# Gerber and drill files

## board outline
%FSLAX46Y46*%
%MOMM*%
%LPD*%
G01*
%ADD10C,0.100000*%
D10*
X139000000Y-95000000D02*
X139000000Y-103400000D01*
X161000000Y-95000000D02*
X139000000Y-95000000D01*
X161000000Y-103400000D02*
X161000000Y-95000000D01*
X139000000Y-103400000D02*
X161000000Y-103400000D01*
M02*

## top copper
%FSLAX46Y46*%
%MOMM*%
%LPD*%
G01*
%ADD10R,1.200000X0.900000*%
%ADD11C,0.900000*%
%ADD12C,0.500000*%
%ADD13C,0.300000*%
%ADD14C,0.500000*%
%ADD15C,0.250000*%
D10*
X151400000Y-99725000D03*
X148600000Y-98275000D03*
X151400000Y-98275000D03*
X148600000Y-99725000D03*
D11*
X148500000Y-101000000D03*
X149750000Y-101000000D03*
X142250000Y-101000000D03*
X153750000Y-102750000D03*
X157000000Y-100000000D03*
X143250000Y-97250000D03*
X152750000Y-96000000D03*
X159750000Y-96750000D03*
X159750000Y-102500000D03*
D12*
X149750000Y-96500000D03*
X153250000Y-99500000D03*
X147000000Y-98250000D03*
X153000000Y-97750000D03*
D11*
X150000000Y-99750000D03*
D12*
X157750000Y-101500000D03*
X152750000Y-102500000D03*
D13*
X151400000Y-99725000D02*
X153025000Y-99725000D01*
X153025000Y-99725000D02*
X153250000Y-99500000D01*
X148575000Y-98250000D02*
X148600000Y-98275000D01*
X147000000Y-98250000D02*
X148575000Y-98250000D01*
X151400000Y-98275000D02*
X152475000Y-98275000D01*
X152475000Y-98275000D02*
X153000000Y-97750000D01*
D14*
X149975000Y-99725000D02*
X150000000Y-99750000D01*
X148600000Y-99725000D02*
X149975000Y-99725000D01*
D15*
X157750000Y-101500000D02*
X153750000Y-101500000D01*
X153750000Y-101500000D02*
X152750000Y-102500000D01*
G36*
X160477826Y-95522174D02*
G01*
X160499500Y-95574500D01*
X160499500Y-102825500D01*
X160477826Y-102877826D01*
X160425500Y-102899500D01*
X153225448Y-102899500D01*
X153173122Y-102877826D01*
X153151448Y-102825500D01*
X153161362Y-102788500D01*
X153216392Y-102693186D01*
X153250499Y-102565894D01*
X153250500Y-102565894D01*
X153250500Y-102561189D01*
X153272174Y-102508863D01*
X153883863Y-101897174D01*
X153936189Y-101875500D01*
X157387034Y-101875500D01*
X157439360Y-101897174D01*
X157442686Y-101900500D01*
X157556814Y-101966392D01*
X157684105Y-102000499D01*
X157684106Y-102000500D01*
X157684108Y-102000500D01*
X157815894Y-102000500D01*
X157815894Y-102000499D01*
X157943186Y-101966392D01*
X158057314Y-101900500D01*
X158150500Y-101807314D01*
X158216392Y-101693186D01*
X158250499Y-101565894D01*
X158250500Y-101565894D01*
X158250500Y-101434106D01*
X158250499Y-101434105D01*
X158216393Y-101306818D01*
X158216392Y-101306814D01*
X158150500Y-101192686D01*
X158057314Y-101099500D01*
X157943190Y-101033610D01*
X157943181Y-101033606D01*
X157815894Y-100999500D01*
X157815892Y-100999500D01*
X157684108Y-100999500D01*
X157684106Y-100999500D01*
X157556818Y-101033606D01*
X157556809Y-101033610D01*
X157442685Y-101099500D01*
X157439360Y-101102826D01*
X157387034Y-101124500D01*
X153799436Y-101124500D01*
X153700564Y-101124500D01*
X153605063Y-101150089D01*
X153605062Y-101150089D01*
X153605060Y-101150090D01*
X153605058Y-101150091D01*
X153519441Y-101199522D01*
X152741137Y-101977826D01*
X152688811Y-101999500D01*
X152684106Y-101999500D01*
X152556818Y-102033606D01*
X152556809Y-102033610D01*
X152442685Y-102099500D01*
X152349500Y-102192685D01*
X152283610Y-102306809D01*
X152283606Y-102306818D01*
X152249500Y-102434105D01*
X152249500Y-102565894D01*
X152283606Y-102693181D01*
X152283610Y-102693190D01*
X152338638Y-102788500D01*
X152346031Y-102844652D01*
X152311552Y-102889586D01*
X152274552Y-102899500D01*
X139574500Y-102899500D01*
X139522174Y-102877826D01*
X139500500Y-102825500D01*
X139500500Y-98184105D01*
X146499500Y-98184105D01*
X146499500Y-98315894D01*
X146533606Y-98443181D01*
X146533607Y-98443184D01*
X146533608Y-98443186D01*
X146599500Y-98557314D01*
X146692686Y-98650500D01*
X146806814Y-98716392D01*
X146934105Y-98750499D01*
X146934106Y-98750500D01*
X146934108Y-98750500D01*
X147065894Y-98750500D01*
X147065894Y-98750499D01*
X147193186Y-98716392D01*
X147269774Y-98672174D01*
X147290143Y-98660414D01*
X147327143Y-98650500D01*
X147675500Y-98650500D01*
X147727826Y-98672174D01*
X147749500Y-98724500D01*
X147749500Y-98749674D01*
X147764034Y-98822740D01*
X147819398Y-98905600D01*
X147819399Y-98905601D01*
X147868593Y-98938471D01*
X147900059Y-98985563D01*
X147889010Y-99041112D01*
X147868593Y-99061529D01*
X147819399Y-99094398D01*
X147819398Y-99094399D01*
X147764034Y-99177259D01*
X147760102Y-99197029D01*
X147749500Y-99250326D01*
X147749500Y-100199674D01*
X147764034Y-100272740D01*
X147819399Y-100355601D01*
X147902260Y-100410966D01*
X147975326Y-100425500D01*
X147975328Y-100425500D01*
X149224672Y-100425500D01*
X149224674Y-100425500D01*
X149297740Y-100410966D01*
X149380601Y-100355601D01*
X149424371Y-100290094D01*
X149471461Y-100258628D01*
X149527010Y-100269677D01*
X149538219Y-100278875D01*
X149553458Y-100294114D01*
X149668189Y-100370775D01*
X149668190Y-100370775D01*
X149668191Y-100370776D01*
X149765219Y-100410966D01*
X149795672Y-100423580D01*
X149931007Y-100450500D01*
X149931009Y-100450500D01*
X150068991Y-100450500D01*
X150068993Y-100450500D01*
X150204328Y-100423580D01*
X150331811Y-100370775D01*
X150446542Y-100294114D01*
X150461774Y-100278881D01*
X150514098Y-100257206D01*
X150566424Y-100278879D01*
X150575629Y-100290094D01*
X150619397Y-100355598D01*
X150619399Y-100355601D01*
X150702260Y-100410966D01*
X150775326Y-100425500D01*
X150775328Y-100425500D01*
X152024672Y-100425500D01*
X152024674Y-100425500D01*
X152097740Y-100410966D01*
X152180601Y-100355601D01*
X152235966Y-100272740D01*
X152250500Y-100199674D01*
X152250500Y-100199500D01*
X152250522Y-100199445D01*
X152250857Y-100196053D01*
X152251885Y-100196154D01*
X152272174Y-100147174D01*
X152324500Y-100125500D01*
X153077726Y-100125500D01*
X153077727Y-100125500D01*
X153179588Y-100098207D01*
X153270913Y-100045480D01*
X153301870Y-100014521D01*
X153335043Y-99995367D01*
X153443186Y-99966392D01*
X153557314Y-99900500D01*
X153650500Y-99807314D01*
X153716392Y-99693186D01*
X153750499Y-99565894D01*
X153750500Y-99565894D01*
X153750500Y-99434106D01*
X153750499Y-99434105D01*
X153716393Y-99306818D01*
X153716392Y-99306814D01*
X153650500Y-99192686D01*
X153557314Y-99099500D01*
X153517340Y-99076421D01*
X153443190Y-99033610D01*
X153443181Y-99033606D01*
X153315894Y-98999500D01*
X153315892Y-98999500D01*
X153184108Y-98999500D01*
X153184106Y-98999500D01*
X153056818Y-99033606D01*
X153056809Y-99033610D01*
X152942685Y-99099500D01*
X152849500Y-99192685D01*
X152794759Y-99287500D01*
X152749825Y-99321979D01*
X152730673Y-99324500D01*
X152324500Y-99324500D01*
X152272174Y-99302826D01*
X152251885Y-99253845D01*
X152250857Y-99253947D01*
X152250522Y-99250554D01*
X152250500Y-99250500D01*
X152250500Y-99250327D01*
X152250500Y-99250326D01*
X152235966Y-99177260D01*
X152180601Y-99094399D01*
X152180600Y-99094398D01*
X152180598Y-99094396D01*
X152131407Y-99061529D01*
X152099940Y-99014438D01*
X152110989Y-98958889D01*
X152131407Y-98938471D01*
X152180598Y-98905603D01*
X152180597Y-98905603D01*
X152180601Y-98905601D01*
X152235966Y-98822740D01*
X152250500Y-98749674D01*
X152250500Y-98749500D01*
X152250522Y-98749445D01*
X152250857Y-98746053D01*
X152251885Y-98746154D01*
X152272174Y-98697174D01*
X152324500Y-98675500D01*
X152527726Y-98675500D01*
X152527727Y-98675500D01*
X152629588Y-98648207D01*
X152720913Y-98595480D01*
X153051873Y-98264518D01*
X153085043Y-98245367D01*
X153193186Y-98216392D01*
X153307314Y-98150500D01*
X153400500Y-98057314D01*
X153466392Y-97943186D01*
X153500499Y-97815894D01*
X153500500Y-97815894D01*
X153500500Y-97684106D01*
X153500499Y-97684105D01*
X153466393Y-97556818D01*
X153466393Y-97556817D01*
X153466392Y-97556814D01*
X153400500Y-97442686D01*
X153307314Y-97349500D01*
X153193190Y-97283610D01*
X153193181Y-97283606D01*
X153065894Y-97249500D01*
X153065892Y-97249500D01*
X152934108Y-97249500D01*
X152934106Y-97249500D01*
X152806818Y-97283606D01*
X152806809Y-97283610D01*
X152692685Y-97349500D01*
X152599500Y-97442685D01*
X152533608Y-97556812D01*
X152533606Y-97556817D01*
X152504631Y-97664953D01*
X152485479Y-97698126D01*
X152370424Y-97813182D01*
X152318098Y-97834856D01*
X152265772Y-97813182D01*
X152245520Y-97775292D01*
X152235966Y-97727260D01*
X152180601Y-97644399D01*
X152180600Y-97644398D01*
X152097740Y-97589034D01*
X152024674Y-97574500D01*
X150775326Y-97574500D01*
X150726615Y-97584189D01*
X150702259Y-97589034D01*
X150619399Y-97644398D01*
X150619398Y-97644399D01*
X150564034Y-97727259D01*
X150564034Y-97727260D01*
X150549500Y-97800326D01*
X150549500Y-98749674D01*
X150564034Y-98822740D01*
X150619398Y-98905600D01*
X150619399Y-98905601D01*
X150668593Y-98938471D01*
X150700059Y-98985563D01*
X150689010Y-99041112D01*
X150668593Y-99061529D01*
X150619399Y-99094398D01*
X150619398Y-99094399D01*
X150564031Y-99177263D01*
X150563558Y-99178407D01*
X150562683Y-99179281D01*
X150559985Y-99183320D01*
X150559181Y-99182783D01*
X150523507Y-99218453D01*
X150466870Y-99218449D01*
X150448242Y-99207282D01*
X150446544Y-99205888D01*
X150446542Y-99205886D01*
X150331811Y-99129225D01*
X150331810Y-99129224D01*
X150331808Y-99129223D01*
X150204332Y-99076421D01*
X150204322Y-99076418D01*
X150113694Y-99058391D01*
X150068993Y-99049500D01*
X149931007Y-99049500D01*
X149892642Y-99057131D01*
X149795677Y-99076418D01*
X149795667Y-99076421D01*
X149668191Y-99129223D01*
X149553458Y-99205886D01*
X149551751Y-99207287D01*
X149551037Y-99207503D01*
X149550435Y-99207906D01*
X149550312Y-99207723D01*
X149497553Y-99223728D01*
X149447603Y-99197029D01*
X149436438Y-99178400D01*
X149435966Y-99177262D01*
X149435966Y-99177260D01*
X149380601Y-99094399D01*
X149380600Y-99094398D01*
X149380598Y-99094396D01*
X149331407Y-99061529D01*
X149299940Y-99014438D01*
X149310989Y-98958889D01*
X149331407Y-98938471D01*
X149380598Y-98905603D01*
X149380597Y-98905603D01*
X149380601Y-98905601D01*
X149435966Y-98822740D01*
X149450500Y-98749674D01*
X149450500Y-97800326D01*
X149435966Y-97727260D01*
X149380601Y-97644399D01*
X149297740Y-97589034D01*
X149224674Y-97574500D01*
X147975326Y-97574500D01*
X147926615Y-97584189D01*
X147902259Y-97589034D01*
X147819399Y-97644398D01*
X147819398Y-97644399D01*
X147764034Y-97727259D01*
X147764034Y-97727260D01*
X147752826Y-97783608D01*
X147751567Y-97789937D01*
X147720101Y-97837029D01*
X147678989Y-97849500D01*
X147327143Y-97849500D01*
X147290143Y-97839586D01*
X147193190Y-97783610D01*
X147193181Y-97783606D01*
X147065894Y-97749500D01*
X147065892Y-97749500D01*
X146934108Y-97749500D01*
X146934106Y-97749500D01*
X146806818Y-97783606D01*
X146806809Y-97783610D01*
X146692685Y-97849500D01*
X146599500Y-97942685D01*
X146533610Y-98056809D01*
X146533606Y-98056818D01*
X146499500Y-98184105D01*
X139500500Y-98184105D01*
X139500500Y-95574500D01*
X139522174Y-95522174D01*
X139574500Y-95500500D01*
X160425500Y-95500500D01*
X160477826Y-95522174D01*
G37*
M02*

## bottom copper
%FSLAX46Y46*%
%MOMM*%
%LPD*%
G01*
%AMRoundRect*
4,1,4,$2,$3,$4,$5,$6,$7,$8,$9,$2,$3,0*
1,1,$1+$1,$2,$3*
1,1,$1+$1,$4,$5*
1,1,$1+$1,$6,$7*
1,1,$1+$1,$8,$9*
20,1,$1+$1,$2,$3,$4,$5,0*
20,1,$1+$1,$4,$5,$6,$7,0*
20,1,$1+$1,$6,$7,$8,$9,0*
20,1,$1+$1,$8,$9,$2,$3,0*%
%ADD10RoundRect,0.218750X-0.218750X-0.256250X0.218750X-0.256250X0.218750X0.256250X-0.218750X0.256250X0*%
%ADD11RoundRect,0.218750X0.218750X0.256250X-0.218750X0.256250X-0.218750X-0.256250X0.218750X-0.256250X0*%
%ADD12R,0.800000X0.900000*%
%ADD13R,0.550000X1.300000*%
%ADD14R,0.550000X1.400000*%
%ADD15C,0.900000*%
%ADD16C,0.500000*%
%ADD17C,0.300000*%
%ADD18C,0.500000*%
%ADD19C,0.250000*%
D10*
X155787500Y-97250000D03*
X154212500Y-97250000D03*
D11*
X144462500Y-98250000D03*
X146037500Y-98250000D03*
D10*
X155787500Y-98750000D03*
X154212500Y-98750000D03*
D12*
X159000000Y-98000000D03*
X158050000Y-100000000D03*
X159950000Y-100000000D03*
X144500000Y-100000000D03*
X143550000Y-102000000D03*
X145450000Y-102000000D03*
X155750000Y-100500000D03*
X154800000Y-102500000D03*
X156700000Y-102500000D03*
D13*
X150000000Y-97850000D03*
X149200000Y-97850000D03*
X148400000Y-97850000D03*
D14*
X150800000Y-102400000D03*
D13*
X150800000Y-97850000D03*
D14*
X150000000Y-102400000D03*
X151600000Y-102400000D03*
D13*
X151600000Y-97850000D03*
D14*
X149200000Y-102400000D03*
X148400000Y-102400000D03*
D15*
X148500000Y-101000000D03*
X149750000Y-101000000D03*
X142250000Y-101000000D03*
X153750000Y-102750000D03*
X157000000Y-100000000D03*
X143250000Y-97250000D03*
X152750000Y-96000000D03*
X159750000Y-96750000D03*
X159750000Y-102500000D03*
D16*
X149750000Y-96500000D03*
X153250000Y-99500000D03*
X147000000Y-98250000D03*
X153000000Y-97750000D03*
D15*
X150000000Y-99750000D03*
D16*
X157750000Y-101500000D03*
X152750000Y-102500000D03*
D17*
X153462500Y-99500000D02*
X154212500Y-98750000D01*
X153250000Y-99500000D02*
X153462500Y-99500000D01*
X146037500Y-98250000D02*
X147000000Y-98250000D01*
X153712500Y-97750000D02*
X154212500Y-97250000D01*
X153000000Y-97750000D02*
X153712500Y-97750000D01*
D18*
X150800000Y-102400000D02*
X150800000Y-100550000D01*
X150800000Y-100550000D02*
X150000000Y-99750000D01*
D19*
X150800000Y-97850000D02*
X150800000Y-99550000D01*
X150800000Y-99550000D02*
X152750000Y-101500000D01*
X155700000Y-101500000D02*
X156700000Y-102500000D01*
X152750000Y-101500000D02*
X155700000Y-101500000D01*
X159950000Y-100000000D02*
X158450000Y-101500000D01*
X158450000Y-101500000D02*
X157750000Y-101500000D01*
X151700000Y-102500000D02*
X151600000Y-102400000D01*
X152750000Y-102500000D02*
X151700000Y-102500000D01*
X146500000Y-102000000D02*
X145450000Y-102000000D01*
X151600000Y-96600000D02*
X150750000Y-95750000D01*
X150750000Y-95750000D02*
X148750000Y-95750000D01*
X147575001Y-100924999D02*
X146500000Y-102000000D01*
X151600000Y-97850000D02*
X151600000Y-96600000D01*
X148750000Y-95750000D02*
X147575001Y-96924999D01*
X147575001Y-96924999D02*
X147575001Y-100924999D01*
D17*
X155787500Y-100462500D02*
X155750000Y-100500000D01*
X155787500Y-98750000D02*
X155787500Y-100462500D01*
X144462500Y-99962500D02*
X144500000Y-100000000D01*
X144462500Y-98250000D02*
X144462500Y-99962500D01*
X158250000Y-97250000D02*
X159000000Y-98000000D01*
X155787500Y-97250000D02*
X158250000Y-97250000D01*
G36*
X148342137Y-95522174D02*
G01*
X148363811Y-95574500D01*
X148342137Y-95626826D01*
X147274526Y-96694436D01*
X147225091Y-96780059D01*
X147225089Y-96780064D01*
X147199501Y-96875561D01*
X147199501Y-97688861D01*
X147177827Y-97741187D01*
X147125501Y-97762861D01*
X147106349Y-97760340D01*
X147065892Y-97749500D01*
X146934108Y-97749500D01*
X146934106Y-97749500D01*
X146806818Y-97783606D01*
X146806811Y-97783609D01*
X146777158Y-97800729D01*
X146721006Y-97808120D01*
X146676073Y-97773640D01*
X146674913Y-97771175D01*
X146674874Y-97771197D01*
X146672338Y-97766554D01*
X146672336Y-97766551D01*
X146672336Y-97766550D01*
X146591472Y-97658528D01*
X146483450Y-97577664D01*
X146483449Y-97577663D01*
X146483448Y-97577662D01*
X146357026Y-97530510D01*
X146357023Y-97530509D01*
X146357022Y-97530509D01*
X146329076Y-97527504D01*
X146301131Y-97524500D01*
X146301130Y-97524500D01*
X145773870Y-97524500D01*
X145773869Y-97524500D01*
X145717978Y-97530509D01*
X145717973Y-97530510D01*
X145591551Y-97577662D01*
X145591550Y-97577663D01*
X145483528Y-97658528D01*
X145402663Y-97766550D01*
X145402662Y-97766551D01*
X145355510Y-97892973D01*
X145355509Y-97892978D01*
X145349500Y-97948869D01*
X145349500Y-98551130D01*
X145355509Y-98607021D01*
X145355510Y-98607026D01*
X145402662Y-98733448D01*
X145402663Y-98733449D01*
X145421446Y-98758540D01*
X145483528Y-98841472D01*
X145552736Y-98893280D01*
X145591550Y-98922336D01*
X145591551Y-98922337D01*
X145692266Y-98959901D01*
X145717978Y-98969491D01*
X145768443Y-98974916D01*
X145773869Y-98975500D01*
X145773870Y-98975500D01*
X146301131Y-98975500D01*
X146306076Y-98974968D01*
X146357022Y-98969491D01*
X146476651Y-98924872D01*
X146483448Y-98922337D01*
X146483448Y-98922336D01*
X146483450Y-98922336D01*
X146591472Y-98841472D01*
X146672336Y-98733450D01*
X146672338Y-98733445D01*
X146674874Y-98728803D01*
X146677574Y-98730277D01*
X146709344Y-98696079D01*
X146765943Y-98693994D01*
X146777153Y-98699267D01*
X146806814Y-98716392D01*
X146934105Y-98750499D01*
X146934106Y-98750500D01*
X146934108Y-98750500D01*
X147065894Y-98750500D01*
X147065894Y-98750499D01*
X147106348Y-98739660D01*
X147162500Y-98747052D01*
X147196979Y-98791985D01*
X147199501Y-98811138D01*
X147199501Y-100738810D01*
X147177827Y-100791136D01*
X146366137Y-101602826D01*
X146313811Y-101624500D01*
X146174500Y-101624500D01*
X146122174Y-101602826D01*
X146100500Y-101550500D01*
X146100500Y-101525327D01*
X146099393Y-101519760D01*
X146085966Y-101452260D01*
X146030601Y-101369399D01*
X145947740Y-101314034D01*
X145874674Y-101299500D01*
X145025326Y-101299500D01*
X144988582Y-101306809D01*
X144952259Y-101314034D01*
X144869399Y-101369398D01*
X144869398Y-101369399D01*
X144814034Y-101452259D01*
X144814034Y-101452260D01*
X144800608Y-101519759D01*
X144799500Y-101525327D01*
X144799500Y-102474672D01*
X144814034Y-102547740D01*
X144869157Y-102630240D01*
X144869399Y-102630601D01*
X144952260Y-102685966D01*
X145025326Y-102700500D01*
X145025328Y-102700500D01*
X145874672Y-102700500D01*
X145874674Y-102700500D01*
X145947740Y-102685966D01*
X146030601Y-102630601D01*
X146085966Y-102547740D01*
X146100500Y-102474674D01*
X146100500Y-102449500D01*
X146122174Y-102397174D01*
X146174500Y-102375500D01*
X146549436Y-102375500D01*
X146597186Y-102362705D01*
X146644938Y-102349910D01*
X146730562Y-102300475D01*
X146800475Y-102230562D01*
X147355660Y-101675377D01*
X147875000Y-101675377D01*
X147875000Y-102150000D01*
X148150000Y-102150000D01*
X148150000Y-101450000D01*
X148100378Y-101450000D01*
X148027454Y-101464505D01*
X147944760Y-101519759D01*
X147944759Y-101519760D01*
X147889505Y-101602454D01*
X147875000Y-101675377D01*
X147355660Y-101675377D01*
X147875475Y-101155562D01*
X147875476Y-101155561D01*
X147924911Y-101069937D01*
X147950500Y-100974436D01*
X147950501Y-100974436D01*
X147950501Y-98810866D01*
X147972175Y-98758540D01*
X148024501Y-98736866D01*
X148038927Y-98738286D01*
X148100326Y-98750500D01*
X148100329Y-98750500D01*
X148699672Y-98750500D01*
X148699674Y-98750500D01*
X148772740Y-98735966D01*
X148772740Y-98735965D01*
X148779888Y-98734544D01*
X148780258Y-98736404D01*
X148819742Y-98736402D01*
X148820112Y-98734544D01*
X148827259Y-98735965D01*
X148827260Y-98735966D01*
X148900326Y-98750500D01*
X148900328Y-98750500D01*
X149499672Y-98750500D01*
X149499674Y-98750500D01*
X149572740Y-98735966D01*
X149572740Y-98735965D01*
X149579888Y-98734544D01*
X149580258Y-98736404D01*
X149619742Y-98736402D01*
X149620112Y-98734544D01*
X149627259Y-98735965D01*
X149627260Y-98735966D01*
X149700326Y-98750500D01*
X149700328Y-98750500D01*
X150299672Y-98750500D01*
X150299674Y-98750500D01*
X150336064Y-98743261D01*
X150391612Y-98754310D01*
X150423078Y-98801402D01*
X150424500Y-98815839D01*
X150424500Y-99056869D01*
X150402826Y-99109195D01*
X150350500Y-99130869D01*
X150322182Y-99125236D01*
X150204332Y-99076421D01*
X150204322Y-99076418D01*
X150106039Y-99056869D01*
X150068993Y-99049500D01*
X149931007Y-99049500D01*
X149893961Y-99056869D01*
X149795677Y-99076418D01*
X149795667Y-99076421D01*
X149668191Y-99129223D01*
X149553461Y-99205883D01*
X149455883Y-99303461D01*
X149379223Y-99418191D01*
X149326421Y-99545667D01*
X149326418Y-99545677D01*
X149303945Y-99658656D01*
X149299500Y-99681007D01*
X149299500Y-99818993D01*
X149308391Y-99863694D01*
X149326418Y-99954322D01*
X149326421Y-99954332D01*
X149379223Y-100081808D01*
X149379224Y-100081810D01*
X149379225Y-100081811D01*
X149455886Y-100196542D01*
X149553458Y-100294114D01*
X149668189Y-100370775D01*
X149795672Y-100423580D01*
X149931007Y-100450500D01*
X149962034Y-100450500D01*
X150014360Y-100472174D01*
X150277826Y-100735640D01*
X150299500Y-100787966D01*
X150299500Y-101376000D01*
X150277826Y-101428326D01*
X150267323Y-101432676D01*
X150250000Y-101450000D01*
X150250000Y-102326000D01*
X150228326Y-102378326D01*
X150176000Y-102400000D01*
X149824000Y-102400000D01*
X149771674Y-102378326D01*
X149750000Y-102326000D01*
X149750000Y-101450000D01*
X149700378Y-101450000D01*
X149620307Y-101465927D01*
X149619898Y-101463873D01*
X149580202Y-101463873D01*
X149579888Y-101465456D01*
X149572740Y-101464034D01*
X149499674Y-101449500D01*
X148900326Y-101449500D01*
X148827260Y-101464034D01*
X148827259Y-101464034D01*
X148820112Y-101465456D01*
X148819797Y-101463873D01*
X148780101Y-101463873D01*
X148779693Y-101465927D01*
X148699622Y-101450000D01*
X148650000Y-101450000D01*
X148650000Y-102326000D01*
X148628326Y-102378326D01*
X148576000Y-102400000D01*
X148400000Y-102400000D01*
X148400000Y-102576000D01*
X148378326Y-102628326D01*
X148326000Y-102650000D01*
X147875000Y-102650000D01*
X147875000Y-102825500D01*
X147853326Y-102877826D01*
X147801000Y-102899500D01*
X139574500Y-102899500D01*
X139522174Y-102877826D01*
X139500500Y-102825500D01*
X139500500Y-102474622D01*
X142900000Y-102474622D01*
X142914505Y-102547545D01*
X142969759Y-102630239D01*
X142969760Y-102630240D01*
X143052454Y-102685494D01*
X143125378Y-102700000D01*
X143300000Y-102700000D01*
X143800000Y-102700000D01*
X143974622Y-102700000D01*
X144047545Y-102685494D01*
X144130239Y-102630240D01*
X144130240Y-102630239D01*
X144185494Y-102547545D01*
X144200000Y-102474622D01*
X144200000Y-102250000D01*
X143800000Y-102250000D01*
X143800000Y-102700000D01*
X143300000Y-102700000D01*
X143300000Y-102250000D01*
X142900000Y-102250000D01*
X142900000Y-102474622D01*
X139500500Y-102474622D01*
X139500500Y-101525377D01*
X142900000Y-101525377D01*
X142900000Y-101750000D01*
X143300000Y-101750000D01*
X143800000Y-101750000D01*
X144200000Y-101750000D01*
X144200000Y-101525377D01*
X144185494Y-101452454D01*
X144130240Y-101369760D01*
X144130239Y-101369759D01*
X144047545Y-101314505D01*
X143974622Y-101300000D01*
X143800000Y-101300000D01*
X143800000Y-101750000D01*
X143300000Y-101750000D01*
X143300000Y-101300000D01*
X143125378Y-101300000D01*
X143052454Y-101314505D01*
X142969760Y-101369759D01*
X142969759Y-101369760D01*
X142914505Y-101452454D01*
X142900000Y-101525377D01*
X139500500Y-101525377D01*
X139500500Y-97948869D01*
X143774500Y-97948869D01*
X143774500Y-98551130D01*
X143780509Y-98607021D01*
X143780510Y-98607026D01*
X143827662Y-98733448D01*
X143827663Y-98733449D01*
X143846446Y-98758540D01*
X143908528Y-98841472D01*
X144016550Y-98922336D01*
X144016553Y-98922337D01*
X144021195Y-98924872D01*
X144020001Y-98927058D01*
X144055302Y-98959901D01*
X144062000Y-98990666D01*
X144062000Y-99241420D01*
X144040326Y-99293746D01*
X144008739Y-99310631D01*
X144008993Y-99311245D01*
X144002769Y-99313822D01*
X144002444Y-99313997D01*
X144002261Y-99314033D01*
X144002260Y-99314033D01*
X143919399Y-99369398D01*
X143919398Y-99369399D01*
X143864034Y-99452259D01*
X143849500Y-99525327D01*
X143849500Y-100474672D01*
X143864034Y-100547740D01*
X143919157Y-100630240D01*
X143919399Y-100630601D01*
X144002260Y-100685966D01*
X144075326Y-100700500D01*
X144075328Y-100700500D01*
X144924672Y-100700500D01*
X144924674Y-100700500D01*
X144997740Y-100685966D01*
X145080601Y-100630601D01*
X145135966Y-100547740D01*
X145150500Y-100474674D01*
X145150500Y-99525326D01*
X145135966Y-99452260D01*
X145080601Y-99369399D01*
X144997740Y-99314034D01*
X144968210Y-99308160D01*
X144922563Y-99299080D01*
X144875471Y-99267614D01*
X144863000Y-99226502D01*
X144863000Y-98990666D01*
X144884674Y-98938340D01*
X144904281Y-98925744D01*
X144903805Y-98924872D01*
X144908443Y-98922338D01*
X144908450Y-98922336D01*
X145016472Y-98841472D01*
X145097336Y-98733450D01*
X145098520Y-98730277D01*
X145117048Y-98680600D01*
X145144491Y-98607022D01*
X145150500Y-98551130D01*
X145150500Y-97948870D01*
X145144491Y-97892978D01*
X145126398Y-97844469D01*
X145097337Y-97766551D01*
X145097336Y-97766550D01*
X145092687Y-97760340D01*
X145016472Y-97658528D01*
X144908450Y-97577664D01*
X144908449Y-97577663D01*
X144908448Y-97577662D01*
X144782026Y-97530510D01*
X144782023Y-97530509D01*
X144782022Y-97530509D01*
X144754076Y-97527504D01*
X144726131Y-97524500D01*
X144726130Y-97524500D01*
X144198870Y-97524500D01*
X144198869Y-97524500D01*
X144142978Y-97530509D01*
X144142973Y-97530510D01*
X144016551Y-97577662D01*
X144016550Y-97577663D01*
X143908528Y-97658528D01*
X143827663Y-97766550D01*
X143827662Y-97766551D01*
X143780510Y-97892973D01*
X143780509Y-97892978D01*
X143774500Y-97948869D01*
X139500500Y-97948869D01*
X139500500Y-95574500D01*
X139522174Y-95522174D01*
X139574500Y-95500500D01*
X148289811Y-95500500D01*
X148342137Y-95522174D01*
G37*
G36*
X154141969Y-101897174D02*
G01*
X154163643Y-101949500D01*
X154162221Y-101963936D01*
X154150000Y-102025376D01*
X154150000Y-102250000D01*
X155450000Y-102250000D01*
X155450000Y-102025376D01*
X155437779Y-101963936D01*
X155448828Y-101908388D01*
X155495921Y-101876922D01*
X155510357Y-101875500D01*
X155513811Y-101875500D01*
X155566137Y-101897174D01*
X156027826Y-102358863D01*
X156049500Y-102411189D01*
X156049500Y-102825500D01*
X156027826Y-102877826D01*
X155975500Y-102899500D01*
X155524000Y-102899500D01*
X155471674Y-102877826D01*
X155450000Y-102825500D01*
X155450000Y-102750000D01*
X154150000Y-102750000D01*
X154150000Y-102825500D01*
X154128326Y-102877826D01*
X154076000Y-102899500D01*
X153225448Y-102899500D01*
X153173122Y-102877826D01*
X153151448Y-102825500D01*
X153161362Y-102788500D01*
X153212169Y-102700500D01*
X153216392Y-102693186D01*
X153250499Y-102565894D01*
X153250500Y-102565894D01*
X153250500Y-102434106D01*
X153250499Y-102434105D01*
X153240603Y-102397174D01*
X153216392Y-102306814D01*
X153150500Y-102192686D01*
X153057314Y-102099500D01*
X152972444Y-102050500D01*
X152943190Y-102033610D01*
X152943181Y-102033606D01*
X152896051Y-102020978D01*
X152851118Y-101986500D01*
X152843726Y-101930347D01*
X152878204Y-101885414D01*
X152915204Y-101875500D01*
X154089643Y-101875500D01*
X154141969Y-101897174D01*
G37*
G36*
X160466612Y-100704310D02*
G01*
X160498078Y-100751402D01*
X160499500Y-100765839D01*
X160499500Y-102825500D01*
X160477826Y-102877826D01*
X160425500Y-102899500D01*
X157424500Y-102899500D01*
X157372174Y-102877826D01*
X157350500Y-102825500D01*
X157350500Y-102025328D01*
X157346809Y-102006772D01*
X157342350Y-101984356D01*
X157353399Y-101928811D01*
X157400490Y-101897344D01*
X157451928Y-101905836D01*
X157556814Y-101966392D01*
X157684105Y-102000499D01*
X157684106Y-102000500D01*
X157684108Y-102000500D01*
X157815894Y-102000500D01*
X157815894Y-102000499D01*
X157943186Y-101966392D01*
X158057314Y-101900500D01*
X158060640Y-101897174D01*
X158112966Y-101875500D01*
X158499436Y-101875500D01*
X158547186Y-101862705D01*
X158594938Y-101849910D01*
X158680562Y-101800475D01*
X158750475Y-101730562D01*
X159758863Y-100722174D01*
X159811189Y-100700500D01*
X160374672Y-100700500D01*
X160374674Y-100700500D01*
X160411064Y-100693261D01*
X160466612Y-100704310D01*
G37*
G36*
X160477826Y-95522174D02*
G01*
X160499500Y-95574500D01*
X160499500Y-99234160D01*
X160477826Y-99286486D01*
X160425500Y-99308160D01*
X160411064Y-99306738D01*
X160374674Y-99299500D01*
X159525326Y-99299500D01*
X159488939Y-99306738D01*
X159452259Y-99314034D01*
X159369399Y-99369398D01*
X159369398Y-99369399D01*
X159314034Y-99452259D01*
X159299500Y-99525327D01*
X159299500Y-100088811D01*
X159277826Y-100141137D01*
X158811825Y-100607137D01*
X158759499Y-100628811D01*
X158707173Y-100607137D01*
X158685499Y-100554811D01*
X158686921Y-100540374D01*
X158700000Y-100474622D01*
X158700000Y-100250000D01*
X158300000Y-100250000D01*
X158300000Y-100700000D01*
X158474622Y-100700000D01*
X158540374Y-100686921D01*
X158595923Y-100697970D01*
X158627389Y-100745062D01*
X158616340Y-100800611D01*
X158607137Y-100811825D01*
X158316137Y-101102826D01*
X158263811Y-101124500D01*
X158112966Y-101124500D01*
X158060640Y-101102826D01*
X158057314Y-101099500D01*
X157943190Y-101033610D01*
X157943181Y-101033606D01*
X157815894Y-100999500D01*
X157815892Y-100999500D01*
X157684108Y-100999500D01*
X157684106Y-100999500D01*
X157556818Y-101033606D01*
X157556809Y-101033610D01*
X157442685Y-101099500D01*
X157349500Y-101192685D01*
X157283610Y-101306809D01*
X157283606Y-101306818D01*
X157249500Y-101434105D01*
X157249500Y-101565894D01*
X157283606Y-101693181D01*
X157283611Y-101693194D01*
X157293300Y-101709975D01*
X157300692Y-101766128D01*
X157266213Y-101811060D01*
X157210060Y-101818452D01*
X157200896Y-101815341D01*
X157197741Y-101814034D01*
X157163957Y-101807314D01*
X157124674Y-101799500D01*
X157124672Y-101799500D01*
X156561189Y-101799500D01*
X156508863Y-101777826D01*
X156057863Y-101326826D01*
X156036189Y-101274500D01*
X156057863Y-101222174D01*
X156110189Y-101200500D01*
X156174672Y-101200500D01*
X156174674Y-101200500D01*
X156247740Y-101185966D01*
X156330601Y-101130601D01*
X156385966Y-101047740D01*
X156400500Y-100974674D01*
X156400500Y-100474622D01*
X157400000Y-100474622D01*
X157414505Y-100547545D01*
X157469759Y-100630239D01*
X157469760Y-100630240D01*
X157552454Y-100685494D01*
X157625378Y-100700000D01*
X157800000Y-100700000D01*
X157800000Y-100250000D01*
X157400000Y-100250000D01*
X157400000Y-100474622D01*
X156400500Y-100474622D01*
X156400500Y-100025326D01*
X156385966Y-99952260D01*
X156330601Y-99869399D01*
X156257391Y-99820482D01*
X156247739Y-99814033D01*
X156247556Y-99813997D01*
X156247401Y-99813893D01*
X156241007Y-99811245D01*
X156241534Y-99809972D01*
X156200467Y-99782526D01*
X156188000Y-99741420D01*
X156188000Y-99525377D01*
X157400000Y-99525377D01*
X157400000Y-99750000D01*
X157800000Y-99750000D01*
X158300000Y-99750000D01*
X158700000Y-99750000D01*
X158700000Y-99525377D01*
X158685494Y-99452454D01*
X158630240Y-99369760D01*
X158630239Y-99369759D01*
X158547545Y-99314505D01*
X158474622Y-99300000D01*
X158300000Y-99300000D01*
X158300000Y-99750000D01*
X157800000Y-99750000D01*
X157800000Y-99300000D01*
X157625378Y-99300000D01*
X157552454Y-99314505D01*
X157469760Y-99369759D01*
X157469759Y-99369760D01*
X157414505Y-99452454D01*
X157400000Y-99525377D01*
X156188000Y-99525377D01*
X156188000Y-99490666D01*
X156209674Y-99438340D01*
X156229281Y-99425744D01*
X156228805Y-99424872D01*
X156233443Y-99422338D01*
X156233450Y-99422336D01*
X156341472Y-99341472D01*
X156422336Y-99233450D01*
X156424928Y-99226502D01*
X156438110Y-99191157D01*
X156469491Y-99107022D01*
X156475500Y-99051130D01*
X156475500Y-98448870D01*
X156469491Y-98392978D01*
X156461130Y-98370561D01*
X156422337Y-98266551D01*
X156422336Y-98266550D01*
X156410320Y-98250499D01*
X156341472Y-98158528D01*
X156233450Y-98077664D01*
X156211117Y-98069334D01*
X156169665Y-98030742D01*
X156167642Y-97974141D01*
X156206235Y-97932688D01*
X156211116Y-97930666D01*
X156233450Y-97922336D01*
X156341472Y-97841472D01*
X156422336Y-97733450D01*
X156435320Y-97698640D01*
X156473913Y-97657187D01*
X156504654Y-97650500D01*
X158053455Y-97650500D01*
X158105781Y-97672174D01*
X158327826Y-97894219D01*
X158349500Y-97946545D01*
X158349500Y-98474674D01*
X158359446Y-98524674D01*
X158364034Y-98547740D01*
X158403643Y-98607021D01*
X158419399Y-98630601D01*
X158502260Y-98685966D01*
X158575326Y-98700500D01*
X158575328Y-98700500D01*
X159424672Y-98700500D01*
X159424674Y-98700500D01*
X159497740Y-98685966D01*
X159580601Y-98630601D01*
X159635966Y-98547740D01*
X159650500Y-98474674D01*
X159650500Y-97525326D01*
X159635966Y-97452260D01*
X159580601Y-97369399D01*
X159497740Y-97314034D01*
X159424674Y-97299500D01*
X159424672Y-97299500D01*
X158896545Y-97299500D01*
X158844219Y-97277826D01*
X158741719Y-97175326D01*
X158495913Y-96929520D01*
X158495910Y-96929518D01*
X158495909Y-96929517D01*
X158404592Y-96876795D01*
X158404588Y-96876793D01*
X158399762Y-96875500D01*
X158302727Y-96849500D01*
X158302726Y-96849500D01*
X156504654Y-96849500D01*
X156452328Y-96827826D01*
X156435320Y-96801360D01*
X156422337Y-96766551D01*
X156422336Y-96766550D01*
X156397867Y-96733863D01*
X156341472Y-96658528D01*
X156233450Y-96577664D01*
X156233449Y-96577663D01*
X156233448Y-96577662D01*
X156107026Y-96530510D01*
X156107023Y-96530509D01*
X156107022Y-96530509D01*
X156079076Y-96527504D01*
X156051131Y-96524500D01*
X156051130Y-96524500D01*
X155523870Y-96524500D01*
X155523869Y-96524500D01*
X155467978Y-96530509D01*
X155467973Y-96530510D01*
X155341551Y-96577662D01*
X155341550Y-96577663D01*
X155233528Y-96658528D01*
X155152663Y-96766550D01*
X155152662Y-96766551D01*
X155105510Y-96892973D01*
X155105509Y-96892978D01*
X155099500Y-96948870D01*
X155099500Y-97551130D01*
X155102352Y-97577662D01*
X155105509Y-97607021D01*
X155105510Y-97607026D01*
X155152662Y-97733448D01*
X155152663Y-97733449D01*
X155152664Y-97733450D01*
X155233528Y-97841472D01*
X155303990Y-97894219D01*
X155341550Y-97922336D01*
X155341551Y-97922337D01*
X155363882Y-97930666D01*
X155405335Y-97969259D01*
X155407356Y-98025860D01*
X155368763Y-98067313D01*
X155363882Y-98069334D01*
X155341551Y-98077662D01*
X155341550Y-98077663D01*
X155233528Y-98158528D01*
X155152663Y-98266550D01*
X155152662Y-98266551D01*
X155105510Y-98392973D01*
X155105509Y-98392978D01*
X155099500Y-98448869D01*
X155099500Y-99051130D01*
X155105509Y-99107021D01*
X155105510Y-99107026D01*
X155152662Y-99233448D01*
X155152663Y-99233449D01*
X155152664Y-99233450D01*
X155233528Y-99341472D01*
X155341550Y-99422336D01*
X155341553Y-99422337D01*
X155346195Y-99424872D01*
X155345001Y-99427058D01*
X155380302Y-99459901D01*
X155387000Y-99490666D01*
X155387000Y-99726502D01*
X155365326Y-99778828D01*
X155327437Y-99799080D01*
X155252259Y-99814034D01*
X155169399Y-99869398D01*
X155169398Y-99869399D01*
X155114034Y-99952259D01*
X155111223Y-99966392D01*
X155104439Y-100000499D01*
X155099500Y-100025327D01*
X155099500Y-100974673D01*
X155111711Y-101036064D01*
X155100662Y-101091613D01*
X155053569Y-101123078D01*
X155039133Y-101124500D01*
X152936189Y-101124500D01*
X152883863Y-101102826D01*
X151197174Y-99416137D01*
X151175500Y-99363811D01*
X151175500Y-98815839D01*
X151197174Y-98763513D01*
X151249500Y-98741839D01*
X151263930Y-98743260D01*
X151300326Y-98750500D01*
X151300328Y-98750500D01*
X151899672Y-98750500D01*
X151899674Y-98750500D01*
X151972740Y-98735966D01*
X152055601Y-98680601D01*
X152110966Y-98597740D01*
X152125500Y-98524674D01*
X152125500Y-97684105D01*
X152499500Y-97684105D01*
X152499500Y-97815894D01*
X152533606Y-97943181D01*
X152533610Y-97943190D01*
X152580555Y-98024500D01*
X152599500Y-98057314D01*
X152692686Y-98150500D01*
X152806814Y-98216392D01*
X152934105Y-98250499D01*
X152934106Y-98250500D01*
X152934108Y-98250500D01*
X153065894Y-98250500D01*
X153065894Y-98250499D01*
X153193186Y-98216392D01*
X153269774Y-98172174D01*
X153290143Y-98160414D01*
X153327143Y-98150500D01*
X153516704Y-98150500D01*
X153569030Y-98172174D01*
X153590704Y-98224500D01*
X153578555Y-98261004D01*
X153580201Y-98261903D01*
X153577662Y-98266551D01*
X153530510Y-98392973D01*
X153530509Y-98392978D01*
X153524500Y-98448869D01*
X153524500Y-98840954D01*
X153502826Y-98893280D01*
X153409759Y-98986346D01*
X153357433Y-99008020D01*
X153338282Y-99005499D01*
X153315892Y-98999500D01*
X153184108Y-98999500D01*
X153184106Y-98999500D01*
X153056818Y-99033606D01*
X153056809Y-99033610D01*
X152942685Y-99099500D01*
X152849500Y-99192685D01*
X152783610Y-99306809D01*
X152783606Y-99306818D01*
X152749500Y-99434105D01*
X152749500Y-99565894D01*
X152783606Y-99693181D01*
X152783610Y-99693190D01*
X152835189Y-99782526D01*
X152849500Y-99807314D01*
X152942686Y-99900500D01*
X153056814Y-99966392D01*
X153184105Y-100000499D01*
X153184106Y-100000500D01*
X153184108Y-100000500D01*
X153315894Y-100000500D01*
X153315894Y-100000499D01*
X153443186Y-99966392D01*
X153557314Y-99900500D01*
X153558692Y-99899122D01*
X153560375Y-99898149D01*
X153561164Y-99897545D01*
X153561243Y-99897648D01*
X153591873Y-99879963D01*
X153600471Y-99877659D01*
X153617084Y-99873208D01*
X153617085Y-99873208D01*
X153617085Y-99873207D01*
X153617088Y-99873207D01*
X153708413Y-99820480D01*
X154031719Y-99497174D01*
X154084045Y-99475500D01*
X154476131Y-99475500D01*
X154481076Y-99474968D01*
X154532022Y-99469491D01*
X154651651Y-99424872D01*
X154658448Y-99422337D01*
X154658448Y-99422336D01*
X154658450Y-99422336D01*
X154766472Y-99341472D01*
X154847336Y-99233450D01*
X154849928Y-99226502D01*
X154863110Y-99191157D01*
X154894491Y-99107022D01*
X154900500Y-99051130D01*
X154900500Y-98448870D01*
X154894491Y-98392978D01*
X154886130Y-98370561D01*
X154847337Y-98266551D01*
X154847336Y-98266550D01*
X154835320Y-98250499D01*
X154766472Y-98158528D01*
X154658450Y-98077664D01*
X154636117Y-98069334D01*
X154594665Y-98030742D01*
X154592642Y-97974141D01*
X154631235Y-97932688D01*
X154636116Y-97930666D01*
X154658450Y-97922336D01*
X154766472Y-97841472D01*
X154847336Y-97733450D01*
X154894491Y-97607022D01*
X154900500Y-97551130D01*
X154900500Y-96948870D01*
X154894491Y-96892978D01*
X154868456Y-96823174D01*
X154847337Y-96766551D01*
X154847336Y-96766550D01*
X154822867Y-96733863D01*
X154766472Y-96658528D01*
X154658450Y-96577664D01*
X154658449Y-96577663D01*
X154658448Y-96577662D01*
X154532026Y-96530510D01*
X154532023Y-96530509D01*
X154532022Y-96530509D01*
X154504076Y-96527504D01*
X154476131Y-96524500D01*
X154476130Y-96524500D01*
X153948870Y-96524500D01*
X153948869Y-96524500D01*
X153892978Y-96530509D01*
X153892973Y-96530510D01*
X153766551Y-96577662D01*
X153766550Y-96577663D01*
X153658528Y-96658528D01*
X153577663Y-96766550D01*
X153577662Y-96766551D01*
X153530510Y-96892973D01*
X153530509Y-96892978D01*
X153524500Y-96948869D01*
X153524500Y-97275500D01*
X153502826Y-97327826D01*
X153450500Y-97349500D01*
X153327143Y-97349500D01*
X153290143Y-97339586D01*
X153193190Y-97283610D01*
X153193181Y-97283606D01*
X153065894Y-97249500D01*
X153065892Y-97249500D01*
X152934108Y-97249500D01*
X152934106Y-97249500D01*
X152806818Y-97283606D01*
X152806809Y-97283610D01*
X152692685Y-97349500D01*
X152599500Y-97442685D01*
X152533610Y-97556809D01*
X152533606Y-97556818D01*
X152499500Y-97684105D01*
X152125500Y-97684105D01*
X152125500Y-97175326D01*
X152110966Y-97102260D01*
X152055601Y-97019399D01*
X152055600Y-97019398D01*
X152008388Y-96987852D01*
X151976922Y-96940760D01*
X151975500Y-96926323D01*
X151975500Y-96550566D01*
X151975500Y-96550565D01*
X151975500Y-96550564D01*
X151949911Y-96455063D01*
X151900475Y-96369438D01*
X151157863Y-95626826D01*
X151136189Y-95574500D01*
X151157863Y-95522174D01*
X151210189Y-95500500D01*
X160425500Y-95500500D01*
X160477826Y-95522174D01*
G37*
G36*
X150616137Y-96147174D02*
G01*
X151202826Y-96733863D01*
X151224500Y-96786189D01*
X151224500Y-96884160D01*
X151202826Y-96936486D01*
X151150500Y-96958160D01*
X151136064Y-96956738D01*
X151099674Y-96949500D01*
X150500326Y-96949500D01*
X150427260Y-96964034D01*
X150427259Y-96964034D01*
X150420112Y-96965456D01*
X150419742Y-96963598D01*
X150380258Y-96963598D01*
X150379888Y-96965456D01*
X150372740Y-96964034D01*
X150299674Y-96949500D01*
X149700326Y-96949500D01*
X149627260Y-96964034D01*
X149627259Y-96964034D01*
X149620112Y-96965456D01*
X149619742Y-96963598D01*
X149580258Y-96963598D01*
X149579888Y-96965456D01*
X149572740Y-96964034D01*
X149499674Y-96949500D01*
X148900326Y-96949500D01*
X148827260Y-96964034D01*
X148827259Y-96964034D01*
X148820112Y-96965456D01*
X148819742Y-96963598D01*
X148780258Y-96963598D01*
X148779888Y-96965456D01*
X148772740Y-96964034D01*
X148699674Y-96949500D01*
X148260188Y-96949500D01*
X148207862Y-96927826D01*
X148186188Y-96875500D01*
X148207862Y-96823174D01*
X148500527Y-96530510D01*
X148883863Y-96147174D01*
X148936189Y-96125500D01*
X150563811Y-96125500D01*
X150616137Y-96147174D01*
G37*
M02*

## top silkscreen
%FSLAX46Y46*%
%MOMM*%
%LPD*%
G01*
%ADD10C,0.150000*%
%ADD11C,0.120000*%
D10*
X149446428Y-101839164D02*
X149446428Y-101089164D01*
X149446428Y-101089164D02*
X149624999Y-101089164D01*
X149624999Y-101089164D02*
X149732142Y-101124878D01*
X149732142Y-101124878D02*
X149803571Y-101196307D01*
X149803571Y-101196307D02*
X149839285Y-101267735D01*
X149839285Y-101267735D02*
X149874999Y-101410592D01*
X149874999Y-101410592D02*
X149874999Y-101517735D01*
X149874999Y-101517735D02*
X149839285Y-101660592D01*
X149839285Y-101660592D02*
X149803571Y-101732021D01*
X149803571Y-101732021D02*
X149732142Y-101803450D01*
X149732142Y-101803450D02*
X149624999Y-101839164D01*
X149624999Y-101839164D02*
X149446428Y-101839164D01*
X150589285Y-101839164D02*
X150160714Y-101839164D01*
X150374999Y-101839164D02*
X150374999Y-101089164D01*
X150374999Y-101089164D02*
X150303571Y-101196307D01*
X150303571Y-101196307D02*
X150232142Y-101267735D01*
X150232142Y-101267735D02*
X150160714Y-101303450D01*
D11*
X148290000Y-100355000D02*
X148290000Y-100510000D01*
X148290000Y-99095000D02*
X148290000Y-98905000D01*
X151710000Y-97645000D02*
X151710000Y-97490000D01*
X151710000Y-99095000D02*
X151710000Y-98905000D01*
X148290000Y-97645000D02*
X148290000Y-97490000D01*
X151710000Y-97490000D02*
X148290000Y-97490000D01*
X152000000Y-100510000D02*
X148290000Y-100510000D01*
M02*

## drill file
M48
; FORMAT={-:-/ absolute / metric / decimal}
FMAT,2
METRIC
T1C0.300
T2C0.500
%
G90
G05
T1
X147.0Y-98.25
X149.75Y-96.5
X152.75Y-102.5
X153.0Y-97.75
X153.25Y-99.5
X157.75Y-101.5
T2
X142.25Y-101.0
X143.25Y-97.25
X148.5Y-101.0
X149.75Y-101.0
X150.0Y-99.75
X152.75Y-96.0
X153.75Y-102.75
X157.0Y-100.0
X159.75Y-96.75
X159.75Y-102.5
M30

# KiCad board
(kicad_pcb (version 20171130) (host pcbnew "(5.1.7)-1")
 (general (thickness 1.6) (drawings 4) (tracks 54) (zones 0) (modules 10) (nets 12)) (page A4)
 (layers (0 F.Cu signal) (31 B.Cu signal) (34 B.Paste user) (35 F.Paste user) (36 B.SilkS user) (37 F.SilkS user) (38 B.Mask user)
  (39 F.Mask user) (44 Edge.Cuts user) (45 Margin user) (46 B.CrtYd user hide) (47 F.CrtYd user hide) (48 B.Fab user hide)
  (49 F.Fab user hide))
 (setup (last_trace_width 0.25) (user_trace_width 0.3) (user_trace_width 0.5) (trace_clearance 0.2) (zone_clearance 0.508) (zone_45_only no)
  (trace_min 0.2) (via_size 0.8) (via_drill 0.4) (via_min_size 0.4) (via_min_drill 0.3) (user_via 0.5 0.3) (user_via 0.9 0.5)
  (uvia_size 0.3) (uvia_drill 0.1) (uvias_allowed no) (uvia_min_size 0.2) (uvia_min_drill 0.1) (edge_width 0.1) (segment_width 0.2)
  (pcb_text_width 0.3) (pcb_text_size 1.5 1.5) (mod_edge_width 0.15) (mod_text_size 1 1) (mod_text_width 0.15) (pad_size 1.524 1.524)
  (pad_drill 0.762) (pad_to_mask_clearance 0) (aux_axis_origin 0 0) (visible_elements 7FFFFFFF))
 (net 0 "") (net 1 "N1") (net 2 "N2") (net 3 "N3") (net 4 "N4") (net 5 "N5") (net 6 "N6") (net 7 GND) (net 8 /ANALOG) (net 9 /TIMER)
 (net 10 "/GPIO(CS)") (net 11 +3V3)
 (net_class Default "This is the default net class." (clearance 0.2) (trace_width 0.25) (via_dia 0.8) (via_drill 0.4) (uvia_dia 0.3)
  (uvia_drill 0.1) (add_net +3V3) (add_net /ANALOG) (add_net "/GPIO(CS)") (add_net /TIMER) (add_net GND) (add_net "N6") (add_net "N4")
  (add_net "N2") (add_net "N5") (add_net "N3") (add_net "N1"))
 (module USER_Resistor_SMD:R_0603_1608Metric (layer B.Cu) (at 155 97.25)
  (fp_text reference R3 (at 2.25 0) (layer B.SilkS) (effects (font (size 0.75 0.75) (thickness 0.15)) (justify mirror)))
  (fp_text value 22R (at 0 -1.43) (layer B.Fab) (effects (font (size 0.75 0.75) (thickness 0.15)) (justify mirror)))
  (pad 2 smd roundrect (at 0.7875 0) (size 0.875 0.95) (layers B.Cu B.Paste B.Mask) (roundrect_rratio 0.25) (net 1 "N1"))
  (pad 1 smd roundrect (at -0.7875 0) (size 0.875 0.95) (layers B.Cu B.Paste B.Mask) (roundrect_rratio 0.25) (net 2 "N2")))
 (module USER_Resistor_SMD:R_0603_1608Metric (layer B.Cu) (at 145.25 98.25 180)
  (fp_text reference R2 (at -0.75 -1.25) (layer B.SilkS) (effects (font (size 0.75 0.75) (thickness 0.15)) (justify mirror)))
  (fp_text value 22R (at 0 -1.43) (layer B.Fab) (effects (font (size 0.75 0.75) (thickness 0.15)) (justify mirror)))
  (pad 2 smd roundrect (at 0.7875 0 180) (size 0.875 0.95) (layers B.Cu B.Paste B.Mask) (roundrect_rratio 0.25) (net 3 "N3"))
  (pad 1 smd roundrect (at -0.7875 0 180) (size 0.875 0.95) (layers B.Cu B.Paste B.Mask) (roundrect_rratio 0.25) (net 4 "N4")))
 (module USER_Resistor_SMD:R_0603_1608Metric (layer B.Cu) (at 155 98.75)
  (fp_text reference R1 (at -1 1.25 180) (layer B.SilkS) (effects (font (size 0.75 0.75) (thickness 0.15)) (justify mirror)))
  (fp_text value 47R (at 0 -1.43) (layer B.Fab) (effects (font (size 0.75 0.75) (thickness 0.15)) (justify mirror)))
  (pad 2 smd roundrect (at 0.7875 0) (size 0.875 0.95) (layers B.Cu B.Paste B.Mask) (roundrect_rratio 0.25) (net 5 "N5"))
  (pad 1 smd roundrect (at -0.7875 0) (size 0.875 0.95) (layers B.Cu B.Paste B.Mask) (roundrect_rratio 0.25) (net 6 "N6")))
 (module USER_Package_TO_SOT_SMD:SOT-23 (layer B.Cu) (at 159 99 90)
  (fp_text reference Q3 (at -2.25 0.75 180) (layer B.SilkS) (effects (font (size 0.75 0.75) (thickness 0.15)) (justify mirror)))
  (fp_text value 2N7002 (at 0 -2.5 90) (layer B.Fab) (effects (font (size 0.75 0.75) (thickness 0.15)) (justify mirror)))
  (pad 3 smd rect (at 1 0 90) (size 0.9 0.8) (layers B.Cu B.Paste B.Mask) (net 1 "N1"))
  (pad 2 smd rect (at -1 -0.95 90) (size 0.9 0.8) (layers B.Cu B.Paste B.Mask) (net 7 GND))
  (pad 1 smd rect (at -1 0.95 90) (size 0.9 0.8) (layers B.Cu B.Paste B.Mask) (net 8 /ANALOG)))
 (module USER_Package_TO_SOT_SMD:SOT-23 (layer B.Cu) (at 144.5 101 90)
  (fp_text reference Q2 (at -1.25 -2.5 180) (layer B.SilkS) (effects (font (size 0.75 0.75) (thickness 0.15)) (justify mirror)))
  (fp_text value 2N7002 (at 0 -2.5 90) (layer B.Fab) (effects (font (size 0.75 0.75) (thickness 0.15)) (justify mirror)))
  (pad 3 smd rect (at 1 0 90) (size 0.9 0.8) (layers B.Cu B.Paste B.Mask) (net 3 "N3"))
  (pad 2 smd rect (at -1 -0.95 90) (size 0.9 0.8) (layers B.Cu B.Paste B.Mask) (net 7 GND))
  (pad 1 smd rect (at -1 0.95 90) (size 0.9 0.8) (layers B.Cu B.Paste B.Mask) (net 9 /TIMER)))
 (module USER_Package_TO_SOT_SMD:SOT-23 (layer B.Cu) (at 155.75 101.5 90)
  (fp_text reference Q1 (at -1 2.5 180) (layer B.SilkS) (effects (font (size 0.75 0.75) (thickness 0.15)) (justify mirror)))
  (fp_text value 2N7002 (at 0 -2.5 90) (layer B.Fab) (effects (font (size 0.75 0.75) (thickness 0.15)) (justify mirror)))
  (pad 3 smd rect (at 1 0 90) (size 0.9 0.8) (layers B.Cu B.Paste B.Mask) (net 5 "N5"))
  (pad 2 smd rect (at -1 -0.95 90) (size 0.9 0.8) (layers B.Cu B.Paste B.Mask) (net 7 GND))
  (pad 1 smd rect (at -1 0.95 90) (size 0.9 0.8) (layers B.Cu B.Paste B.Mask) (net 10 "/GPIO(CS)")))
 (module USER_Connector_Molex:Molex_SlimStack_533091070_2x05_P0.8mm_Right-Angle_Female (layer B.Cu) (at 150 100)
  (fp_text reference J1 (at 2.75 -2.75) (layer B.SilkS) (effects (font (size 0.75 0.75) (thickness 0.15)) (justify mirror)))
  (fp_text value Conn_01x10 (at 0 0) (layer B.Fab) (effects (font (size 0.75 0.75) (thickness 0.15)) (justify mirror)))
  (pad 5 smd rect (at 0 -2.15 180) (size 0.55 1.3) (layers B.Cu B.Paste B.Mask))
  (pad 3 smd rect (at -0.8 -2.15 180) (size 0.55 1.3) (layers B.Cu B.Paste B.Mask))
  (pad 1 smd rect (at -1.6 -2.15 180) (size 0.55 1.3) (layers B.Cu B.Paste B.Mask))
  (pad 8 smd rect (at 0.8 2.4 180) (size 0.55 1.4) (layers B.Cu B.Paste B.Mask) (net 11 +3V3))
  (pad 7 smd rect (at 0.8 -2.15 180) (size 0.55 1.3) (layers B.Cu B.Paste B.Mask) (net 10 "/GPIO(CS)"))
  (pad 6 smd rect (at 0 2.4 180) (size 0.55 1.4) (layers B.Cu B.Paste B.Mask) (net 7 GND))
  (pad 10 smd rect (at 1.6 2.4 180) (size 0.55 1.4) (layers B.Cu B.Paste B.Mask) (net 8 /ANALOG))
  (pad 9 smd rect (at 1.6 -2.15 180) (size 0.55 1.3) (layers B.Cu B.Paste B.Mask) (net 9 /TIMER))
  (pad 4 smd rect (at -0.8 2.4 180) (size 0.55 1.4) (layers B.Cu B.Paste B.Mask))
  (pad 2 smd rect (at -1.6 2.4 180) (size 0.55 1.4) (layers B.Cu B.Paste B.Mask) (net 7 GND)))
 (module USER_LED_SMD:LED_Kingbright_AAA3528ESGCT (layer F.Cu) (at 150 99 180)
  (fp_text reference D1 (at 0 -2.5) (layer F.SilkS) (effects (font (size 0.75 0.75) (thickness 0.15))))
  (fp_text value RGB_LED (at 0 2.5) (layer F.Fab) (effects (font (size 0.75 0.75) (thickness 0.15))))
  (fp_line (start 1.71 -1.355) (end 1.71 -1.51) (layer F.SilkS) (width 0.12))
  (fp_line (start 1.71 -0.095) (end 1.71 0.095) (layer F.SilkS) (width 0.12))
  (fp_line (start -1.71 1.355) (end -1.71 1.51) (layer F.SilkS) (width 0.12))
  (fp_line (start -1.71 -0.095) (end -1.71 0.095) (layer F.SilkS) (width 0.12))
  (fp_line (start 1.71 1.355) (end 1.71 1.51) (layer F.SilkS) (width 0.12))
  (fp_line (start -1.71 1.51) (end 1.71 1.51) (layer F.SilkS) (width 0.12))
  (fp_line (start -2 -1.51) (end 1.71 -1.51) (layer F.SilkS) (width 0.12))
  (pad 1 smd rect (at -1.4 -0.725 180) (size 1.2 0.9) (layers F.Cu F.Paste F.Mask) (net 6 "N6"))
  (pad 3 smd rect (at 1.4 0.725 180) (size 1.2 0.9) (layers F.Cu F.Paste F.Mask) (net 4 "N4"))
  (pad 4 smd rect (at -1.4 0.725 180) (size 1.2 0.9) (layers F.Cu F.Paste F.Mask) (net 2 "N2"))
  (pad 2 smd rect (at 1.4 -0.725 180) (size 1.2 0.9) (layers F.Cu F.Paste F.Mask) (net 11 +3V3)))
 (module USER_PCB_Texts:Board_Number (layer B.Cu) (at 138.9 97.4)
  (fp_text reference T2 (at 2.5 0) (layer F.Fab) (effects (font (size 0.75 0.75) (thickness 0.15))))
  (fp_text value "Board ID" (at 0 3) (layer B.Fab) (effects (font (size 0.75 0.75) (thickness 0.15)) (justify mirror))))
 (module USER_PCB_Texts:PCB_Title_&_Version (layer F.Cu) (at 147.594999 110.734999)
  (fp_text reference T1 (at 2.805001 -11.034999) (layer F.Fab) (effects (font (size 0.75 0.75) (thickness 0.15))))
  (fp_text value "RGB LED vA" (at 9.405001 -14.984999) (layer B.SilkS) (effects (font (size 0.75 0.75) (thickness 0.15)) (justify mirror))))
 (gr_line (start 139 95) (end 139 103.4) (layer Edge.Cuts) (width 0.1))
 (gr_line (start 161 95) (end 139 95) (layer Edge.Cuts) (width 0.1))
 (gr_line (start 161 103.4) (end 161 95) (layer Edge.Cuts) (width 0.1))
 (gr_line (start 139 103.4) (end 161 103.4) (layer Edge.Cuts) (width 0.1))
 (via (at 148.5 101) (size 0.9) (drill 0.5) (layers F.Cu B.Cu) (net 7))
 (via (at 149.75 101) (size 0.9) (drill 0.5) (layers F.Cu B.Cu) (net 7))
 (via (at 142.25 101) (size 0.9) (drill 0.5) (layers F.Cu B.Cu) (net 7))
 (via (at 153.75 102.75) (size 0.9) (drill 0.5) (layers F.Cu B.Cu) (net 7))
 (via (at 157 100) (size 0.9) (drill 0.5) (layers F.Cu B.Cu) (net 7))
 (via (at 143.25 97.25) (size 0.9) (drill 0.5) (layers F.Cu B.Cu) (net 7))
 (via (at 152.75 96) (size 0.9) (drill 0.5) (layers F.Cu B.Cu) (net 7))
 (via (at 159.75 96.75) (size 0.9) (drill 0.5) (layers F.Cu B.Cu) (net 7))
 (via (at 159.75 102.5) (size 0.9) (drill 0.5) (layers F.Cu B.Cu) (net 7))
 (via (at 149.75 96.5) (size 0.5) (drill 0.3) (layers F.Cu B.Cu) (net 7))
 (via (at 153.25 99.5) (size 0.5) (drill 0.3) (layers F.Cu B.Cu) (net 6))
 (segment (start 151.4 99.725) (end 153.025 99.725) (width 0.3) (layer F.Cu) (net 6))
 (segment (start 153.025 99.725) (end 153.25 99.5) (width 0.3) (layer F.Cu) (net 6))
 (segment (start 153.4625 99.5) (end 154.2125 98.75) (width 0.3) (layer B.Cu) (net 6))
 (segment (start 153.25 99.5) (end 153.4625 99.5) (width 0.3) (layer B.Cu) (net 6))
 (via (at 147 98.25) (size 0.5) (drill 0.3) (layers F.Cu B.Cu) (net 4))
 (segment (start 146.0375 98.25) (end 147 98.25) (width 0.3) (layer B.Cu) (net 4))
 (segment (start 148.575 98.25) (end 148.6 98.275) (width 0.3) (layer F.Cu) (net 4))
 (segment (start 147 98.25) (end 148.575 98.25) (width 0.3) (layer F.Cu) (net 4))
 (segment (start 151.4 98.275) (end 152.475 98.275) (width 0.3) (layer F.Cu) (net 2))
 (via (at 153 97.75) (size 0.5) (drill 0.3) (layers F.Cu B.Cu) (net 2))
 (segment (start 152.475 98.275) (end 153 97.75) (width 0.3) (layer F.Cu) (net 2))
 (segment (start 153.7125 97.75) (end 154.2125 97.25) (width 0.3) (layer B.Cu) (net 2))
 (segment (start 153 97.75) (end 153.7125 97.75) (width 0.3) (layer B.Cu) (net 2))
 (segment (start 150.8 102.4) (end 150.8 100.55) (width 0.5) (layer B.Cu) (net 11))
 (segment (start 149.975 99.725) (end 150 99.75) (width 0.5) (layer F.Cu) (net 11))
 (via (at 150 99.75) (size 0.9) (drill 0.5) (layers F.Cu B.Cu) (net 11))
 (segment (start 150.8 100.55) (end 150 99.75) (width 0.5) (layer B.Cu) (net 11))
 (segment (start 148.6 99.725) (end 149.975 99.725) (width 0.5) (layer F.Cu) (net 11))
 (segment (start 150.8 97.85) (end 150.8 99.55) (width 0.25) (layer B.Cu) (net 10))
 (segment (start 150.8 99.55) (end 152.75 101.5) (width 0.25) (layer B.Cu) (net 10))
 (segment (start 155.7 101.5) (end 156.7 102.5) (width 0.25) (layer B.Cu) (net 10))
 (segment (start 152.75 101.5) (end 155.7 101.5) (width 0.25) (layer B.Cu) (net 10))
 (via (at 157.75 101.5) (size 0.5) (drill 0.3) (layers F.Cu B.Cu) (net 8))
 (segment (start 159.95 100) (end 158.45 101.5) (width 0.25) (layer B.Cu) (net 8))
 (segment (start 158.45 101.5) (end 157.75 101.5) (width 0.25) (layer B.Cu) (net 8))
 (via (at 152.75 102.5) (size 0.5) (drill 0.3) (layers F.Cu B.Cu) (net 8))
 (segment (start 157.75 101.5) (end 153.75 101.5) (width 0.25) (layer F.Cu) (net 8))
 (segment (start 153.75 101.5) (end 152.75 102.5) (width 0.25) (layer F.Cu) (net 8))
 (segment (start 151.7 102.5) (end 151.6 102.4) (width 0.25) (layer B.Cu) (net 8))
 (segment (start 152.75 102.5) (end 151.7 102.5) (width 0.25) (layer B.Cu) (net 8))
 (segment (start 146.5 102) (end 145.45 102) (width 0.25) (layer B.Cu) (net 9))
 (segment (start 151.6 96.6) (end 150.75 95.75) (width 0.25) (layer B.Cu) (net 9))
 (segment (start 150.75 95.75) (end 148.75 95.75) (width 0.25) (layer B.Cu) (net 9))
 (segment (start 147.575001 100.924999) (end 146.5 102) (width 0.25) (layer B.Cu) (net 9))
 (segment (start 151.6 97.85) (end 151.6 96.6) (width 0.25) (layer B.Cu) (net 9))
 (segment (start 148.75 95.75) (end 147.575001 96.924999) (width 0.25) (layer B.Cu) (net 9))
 (segment (start 147.575001 96.924999) (end 147.575001 100.924999) (width 0.25) (layer B.Cu) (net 9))
 (segment (start 155.7875 100.4625) (end 155.75 100.5) (width 0.3) (layer B.Cu) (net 5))
 (segment (start 155.7875 98.75) (end 155.7875 100.4625) (width 0.3) (layer B.Cu) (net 5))
 (segment (start 144.4625 99.9625) (end 144.5 100) (width 0.3) (layer B.Cu) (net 3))
 (segment (start 144.4625 98.25) (end 144.4625 99.9625) (width 0.3) (layer B.Cu) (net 3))
 (segment (start 158.25 97.25) (end 159 98) (width 0.3) (layer B.Cu) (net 1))
 (segment (start 155.7875 97.25) (end 158.25 97.25) (width 0.3) (layer B.Cu) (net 1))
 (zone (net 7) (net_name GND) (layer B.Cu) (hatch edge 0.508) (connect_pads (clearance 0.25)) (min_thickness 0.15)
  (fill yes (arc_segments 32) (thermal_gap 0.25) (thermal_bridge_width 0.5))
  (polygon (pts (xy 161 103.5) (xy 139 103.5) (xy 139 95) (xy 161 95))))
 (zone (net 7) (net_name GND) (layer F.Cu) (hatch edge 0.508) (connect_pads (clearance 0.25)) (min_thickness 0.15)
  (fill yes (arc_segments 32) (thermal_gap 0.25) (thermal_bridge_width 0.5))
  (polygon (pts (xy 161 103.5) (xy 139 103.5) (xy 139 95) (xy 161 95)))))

